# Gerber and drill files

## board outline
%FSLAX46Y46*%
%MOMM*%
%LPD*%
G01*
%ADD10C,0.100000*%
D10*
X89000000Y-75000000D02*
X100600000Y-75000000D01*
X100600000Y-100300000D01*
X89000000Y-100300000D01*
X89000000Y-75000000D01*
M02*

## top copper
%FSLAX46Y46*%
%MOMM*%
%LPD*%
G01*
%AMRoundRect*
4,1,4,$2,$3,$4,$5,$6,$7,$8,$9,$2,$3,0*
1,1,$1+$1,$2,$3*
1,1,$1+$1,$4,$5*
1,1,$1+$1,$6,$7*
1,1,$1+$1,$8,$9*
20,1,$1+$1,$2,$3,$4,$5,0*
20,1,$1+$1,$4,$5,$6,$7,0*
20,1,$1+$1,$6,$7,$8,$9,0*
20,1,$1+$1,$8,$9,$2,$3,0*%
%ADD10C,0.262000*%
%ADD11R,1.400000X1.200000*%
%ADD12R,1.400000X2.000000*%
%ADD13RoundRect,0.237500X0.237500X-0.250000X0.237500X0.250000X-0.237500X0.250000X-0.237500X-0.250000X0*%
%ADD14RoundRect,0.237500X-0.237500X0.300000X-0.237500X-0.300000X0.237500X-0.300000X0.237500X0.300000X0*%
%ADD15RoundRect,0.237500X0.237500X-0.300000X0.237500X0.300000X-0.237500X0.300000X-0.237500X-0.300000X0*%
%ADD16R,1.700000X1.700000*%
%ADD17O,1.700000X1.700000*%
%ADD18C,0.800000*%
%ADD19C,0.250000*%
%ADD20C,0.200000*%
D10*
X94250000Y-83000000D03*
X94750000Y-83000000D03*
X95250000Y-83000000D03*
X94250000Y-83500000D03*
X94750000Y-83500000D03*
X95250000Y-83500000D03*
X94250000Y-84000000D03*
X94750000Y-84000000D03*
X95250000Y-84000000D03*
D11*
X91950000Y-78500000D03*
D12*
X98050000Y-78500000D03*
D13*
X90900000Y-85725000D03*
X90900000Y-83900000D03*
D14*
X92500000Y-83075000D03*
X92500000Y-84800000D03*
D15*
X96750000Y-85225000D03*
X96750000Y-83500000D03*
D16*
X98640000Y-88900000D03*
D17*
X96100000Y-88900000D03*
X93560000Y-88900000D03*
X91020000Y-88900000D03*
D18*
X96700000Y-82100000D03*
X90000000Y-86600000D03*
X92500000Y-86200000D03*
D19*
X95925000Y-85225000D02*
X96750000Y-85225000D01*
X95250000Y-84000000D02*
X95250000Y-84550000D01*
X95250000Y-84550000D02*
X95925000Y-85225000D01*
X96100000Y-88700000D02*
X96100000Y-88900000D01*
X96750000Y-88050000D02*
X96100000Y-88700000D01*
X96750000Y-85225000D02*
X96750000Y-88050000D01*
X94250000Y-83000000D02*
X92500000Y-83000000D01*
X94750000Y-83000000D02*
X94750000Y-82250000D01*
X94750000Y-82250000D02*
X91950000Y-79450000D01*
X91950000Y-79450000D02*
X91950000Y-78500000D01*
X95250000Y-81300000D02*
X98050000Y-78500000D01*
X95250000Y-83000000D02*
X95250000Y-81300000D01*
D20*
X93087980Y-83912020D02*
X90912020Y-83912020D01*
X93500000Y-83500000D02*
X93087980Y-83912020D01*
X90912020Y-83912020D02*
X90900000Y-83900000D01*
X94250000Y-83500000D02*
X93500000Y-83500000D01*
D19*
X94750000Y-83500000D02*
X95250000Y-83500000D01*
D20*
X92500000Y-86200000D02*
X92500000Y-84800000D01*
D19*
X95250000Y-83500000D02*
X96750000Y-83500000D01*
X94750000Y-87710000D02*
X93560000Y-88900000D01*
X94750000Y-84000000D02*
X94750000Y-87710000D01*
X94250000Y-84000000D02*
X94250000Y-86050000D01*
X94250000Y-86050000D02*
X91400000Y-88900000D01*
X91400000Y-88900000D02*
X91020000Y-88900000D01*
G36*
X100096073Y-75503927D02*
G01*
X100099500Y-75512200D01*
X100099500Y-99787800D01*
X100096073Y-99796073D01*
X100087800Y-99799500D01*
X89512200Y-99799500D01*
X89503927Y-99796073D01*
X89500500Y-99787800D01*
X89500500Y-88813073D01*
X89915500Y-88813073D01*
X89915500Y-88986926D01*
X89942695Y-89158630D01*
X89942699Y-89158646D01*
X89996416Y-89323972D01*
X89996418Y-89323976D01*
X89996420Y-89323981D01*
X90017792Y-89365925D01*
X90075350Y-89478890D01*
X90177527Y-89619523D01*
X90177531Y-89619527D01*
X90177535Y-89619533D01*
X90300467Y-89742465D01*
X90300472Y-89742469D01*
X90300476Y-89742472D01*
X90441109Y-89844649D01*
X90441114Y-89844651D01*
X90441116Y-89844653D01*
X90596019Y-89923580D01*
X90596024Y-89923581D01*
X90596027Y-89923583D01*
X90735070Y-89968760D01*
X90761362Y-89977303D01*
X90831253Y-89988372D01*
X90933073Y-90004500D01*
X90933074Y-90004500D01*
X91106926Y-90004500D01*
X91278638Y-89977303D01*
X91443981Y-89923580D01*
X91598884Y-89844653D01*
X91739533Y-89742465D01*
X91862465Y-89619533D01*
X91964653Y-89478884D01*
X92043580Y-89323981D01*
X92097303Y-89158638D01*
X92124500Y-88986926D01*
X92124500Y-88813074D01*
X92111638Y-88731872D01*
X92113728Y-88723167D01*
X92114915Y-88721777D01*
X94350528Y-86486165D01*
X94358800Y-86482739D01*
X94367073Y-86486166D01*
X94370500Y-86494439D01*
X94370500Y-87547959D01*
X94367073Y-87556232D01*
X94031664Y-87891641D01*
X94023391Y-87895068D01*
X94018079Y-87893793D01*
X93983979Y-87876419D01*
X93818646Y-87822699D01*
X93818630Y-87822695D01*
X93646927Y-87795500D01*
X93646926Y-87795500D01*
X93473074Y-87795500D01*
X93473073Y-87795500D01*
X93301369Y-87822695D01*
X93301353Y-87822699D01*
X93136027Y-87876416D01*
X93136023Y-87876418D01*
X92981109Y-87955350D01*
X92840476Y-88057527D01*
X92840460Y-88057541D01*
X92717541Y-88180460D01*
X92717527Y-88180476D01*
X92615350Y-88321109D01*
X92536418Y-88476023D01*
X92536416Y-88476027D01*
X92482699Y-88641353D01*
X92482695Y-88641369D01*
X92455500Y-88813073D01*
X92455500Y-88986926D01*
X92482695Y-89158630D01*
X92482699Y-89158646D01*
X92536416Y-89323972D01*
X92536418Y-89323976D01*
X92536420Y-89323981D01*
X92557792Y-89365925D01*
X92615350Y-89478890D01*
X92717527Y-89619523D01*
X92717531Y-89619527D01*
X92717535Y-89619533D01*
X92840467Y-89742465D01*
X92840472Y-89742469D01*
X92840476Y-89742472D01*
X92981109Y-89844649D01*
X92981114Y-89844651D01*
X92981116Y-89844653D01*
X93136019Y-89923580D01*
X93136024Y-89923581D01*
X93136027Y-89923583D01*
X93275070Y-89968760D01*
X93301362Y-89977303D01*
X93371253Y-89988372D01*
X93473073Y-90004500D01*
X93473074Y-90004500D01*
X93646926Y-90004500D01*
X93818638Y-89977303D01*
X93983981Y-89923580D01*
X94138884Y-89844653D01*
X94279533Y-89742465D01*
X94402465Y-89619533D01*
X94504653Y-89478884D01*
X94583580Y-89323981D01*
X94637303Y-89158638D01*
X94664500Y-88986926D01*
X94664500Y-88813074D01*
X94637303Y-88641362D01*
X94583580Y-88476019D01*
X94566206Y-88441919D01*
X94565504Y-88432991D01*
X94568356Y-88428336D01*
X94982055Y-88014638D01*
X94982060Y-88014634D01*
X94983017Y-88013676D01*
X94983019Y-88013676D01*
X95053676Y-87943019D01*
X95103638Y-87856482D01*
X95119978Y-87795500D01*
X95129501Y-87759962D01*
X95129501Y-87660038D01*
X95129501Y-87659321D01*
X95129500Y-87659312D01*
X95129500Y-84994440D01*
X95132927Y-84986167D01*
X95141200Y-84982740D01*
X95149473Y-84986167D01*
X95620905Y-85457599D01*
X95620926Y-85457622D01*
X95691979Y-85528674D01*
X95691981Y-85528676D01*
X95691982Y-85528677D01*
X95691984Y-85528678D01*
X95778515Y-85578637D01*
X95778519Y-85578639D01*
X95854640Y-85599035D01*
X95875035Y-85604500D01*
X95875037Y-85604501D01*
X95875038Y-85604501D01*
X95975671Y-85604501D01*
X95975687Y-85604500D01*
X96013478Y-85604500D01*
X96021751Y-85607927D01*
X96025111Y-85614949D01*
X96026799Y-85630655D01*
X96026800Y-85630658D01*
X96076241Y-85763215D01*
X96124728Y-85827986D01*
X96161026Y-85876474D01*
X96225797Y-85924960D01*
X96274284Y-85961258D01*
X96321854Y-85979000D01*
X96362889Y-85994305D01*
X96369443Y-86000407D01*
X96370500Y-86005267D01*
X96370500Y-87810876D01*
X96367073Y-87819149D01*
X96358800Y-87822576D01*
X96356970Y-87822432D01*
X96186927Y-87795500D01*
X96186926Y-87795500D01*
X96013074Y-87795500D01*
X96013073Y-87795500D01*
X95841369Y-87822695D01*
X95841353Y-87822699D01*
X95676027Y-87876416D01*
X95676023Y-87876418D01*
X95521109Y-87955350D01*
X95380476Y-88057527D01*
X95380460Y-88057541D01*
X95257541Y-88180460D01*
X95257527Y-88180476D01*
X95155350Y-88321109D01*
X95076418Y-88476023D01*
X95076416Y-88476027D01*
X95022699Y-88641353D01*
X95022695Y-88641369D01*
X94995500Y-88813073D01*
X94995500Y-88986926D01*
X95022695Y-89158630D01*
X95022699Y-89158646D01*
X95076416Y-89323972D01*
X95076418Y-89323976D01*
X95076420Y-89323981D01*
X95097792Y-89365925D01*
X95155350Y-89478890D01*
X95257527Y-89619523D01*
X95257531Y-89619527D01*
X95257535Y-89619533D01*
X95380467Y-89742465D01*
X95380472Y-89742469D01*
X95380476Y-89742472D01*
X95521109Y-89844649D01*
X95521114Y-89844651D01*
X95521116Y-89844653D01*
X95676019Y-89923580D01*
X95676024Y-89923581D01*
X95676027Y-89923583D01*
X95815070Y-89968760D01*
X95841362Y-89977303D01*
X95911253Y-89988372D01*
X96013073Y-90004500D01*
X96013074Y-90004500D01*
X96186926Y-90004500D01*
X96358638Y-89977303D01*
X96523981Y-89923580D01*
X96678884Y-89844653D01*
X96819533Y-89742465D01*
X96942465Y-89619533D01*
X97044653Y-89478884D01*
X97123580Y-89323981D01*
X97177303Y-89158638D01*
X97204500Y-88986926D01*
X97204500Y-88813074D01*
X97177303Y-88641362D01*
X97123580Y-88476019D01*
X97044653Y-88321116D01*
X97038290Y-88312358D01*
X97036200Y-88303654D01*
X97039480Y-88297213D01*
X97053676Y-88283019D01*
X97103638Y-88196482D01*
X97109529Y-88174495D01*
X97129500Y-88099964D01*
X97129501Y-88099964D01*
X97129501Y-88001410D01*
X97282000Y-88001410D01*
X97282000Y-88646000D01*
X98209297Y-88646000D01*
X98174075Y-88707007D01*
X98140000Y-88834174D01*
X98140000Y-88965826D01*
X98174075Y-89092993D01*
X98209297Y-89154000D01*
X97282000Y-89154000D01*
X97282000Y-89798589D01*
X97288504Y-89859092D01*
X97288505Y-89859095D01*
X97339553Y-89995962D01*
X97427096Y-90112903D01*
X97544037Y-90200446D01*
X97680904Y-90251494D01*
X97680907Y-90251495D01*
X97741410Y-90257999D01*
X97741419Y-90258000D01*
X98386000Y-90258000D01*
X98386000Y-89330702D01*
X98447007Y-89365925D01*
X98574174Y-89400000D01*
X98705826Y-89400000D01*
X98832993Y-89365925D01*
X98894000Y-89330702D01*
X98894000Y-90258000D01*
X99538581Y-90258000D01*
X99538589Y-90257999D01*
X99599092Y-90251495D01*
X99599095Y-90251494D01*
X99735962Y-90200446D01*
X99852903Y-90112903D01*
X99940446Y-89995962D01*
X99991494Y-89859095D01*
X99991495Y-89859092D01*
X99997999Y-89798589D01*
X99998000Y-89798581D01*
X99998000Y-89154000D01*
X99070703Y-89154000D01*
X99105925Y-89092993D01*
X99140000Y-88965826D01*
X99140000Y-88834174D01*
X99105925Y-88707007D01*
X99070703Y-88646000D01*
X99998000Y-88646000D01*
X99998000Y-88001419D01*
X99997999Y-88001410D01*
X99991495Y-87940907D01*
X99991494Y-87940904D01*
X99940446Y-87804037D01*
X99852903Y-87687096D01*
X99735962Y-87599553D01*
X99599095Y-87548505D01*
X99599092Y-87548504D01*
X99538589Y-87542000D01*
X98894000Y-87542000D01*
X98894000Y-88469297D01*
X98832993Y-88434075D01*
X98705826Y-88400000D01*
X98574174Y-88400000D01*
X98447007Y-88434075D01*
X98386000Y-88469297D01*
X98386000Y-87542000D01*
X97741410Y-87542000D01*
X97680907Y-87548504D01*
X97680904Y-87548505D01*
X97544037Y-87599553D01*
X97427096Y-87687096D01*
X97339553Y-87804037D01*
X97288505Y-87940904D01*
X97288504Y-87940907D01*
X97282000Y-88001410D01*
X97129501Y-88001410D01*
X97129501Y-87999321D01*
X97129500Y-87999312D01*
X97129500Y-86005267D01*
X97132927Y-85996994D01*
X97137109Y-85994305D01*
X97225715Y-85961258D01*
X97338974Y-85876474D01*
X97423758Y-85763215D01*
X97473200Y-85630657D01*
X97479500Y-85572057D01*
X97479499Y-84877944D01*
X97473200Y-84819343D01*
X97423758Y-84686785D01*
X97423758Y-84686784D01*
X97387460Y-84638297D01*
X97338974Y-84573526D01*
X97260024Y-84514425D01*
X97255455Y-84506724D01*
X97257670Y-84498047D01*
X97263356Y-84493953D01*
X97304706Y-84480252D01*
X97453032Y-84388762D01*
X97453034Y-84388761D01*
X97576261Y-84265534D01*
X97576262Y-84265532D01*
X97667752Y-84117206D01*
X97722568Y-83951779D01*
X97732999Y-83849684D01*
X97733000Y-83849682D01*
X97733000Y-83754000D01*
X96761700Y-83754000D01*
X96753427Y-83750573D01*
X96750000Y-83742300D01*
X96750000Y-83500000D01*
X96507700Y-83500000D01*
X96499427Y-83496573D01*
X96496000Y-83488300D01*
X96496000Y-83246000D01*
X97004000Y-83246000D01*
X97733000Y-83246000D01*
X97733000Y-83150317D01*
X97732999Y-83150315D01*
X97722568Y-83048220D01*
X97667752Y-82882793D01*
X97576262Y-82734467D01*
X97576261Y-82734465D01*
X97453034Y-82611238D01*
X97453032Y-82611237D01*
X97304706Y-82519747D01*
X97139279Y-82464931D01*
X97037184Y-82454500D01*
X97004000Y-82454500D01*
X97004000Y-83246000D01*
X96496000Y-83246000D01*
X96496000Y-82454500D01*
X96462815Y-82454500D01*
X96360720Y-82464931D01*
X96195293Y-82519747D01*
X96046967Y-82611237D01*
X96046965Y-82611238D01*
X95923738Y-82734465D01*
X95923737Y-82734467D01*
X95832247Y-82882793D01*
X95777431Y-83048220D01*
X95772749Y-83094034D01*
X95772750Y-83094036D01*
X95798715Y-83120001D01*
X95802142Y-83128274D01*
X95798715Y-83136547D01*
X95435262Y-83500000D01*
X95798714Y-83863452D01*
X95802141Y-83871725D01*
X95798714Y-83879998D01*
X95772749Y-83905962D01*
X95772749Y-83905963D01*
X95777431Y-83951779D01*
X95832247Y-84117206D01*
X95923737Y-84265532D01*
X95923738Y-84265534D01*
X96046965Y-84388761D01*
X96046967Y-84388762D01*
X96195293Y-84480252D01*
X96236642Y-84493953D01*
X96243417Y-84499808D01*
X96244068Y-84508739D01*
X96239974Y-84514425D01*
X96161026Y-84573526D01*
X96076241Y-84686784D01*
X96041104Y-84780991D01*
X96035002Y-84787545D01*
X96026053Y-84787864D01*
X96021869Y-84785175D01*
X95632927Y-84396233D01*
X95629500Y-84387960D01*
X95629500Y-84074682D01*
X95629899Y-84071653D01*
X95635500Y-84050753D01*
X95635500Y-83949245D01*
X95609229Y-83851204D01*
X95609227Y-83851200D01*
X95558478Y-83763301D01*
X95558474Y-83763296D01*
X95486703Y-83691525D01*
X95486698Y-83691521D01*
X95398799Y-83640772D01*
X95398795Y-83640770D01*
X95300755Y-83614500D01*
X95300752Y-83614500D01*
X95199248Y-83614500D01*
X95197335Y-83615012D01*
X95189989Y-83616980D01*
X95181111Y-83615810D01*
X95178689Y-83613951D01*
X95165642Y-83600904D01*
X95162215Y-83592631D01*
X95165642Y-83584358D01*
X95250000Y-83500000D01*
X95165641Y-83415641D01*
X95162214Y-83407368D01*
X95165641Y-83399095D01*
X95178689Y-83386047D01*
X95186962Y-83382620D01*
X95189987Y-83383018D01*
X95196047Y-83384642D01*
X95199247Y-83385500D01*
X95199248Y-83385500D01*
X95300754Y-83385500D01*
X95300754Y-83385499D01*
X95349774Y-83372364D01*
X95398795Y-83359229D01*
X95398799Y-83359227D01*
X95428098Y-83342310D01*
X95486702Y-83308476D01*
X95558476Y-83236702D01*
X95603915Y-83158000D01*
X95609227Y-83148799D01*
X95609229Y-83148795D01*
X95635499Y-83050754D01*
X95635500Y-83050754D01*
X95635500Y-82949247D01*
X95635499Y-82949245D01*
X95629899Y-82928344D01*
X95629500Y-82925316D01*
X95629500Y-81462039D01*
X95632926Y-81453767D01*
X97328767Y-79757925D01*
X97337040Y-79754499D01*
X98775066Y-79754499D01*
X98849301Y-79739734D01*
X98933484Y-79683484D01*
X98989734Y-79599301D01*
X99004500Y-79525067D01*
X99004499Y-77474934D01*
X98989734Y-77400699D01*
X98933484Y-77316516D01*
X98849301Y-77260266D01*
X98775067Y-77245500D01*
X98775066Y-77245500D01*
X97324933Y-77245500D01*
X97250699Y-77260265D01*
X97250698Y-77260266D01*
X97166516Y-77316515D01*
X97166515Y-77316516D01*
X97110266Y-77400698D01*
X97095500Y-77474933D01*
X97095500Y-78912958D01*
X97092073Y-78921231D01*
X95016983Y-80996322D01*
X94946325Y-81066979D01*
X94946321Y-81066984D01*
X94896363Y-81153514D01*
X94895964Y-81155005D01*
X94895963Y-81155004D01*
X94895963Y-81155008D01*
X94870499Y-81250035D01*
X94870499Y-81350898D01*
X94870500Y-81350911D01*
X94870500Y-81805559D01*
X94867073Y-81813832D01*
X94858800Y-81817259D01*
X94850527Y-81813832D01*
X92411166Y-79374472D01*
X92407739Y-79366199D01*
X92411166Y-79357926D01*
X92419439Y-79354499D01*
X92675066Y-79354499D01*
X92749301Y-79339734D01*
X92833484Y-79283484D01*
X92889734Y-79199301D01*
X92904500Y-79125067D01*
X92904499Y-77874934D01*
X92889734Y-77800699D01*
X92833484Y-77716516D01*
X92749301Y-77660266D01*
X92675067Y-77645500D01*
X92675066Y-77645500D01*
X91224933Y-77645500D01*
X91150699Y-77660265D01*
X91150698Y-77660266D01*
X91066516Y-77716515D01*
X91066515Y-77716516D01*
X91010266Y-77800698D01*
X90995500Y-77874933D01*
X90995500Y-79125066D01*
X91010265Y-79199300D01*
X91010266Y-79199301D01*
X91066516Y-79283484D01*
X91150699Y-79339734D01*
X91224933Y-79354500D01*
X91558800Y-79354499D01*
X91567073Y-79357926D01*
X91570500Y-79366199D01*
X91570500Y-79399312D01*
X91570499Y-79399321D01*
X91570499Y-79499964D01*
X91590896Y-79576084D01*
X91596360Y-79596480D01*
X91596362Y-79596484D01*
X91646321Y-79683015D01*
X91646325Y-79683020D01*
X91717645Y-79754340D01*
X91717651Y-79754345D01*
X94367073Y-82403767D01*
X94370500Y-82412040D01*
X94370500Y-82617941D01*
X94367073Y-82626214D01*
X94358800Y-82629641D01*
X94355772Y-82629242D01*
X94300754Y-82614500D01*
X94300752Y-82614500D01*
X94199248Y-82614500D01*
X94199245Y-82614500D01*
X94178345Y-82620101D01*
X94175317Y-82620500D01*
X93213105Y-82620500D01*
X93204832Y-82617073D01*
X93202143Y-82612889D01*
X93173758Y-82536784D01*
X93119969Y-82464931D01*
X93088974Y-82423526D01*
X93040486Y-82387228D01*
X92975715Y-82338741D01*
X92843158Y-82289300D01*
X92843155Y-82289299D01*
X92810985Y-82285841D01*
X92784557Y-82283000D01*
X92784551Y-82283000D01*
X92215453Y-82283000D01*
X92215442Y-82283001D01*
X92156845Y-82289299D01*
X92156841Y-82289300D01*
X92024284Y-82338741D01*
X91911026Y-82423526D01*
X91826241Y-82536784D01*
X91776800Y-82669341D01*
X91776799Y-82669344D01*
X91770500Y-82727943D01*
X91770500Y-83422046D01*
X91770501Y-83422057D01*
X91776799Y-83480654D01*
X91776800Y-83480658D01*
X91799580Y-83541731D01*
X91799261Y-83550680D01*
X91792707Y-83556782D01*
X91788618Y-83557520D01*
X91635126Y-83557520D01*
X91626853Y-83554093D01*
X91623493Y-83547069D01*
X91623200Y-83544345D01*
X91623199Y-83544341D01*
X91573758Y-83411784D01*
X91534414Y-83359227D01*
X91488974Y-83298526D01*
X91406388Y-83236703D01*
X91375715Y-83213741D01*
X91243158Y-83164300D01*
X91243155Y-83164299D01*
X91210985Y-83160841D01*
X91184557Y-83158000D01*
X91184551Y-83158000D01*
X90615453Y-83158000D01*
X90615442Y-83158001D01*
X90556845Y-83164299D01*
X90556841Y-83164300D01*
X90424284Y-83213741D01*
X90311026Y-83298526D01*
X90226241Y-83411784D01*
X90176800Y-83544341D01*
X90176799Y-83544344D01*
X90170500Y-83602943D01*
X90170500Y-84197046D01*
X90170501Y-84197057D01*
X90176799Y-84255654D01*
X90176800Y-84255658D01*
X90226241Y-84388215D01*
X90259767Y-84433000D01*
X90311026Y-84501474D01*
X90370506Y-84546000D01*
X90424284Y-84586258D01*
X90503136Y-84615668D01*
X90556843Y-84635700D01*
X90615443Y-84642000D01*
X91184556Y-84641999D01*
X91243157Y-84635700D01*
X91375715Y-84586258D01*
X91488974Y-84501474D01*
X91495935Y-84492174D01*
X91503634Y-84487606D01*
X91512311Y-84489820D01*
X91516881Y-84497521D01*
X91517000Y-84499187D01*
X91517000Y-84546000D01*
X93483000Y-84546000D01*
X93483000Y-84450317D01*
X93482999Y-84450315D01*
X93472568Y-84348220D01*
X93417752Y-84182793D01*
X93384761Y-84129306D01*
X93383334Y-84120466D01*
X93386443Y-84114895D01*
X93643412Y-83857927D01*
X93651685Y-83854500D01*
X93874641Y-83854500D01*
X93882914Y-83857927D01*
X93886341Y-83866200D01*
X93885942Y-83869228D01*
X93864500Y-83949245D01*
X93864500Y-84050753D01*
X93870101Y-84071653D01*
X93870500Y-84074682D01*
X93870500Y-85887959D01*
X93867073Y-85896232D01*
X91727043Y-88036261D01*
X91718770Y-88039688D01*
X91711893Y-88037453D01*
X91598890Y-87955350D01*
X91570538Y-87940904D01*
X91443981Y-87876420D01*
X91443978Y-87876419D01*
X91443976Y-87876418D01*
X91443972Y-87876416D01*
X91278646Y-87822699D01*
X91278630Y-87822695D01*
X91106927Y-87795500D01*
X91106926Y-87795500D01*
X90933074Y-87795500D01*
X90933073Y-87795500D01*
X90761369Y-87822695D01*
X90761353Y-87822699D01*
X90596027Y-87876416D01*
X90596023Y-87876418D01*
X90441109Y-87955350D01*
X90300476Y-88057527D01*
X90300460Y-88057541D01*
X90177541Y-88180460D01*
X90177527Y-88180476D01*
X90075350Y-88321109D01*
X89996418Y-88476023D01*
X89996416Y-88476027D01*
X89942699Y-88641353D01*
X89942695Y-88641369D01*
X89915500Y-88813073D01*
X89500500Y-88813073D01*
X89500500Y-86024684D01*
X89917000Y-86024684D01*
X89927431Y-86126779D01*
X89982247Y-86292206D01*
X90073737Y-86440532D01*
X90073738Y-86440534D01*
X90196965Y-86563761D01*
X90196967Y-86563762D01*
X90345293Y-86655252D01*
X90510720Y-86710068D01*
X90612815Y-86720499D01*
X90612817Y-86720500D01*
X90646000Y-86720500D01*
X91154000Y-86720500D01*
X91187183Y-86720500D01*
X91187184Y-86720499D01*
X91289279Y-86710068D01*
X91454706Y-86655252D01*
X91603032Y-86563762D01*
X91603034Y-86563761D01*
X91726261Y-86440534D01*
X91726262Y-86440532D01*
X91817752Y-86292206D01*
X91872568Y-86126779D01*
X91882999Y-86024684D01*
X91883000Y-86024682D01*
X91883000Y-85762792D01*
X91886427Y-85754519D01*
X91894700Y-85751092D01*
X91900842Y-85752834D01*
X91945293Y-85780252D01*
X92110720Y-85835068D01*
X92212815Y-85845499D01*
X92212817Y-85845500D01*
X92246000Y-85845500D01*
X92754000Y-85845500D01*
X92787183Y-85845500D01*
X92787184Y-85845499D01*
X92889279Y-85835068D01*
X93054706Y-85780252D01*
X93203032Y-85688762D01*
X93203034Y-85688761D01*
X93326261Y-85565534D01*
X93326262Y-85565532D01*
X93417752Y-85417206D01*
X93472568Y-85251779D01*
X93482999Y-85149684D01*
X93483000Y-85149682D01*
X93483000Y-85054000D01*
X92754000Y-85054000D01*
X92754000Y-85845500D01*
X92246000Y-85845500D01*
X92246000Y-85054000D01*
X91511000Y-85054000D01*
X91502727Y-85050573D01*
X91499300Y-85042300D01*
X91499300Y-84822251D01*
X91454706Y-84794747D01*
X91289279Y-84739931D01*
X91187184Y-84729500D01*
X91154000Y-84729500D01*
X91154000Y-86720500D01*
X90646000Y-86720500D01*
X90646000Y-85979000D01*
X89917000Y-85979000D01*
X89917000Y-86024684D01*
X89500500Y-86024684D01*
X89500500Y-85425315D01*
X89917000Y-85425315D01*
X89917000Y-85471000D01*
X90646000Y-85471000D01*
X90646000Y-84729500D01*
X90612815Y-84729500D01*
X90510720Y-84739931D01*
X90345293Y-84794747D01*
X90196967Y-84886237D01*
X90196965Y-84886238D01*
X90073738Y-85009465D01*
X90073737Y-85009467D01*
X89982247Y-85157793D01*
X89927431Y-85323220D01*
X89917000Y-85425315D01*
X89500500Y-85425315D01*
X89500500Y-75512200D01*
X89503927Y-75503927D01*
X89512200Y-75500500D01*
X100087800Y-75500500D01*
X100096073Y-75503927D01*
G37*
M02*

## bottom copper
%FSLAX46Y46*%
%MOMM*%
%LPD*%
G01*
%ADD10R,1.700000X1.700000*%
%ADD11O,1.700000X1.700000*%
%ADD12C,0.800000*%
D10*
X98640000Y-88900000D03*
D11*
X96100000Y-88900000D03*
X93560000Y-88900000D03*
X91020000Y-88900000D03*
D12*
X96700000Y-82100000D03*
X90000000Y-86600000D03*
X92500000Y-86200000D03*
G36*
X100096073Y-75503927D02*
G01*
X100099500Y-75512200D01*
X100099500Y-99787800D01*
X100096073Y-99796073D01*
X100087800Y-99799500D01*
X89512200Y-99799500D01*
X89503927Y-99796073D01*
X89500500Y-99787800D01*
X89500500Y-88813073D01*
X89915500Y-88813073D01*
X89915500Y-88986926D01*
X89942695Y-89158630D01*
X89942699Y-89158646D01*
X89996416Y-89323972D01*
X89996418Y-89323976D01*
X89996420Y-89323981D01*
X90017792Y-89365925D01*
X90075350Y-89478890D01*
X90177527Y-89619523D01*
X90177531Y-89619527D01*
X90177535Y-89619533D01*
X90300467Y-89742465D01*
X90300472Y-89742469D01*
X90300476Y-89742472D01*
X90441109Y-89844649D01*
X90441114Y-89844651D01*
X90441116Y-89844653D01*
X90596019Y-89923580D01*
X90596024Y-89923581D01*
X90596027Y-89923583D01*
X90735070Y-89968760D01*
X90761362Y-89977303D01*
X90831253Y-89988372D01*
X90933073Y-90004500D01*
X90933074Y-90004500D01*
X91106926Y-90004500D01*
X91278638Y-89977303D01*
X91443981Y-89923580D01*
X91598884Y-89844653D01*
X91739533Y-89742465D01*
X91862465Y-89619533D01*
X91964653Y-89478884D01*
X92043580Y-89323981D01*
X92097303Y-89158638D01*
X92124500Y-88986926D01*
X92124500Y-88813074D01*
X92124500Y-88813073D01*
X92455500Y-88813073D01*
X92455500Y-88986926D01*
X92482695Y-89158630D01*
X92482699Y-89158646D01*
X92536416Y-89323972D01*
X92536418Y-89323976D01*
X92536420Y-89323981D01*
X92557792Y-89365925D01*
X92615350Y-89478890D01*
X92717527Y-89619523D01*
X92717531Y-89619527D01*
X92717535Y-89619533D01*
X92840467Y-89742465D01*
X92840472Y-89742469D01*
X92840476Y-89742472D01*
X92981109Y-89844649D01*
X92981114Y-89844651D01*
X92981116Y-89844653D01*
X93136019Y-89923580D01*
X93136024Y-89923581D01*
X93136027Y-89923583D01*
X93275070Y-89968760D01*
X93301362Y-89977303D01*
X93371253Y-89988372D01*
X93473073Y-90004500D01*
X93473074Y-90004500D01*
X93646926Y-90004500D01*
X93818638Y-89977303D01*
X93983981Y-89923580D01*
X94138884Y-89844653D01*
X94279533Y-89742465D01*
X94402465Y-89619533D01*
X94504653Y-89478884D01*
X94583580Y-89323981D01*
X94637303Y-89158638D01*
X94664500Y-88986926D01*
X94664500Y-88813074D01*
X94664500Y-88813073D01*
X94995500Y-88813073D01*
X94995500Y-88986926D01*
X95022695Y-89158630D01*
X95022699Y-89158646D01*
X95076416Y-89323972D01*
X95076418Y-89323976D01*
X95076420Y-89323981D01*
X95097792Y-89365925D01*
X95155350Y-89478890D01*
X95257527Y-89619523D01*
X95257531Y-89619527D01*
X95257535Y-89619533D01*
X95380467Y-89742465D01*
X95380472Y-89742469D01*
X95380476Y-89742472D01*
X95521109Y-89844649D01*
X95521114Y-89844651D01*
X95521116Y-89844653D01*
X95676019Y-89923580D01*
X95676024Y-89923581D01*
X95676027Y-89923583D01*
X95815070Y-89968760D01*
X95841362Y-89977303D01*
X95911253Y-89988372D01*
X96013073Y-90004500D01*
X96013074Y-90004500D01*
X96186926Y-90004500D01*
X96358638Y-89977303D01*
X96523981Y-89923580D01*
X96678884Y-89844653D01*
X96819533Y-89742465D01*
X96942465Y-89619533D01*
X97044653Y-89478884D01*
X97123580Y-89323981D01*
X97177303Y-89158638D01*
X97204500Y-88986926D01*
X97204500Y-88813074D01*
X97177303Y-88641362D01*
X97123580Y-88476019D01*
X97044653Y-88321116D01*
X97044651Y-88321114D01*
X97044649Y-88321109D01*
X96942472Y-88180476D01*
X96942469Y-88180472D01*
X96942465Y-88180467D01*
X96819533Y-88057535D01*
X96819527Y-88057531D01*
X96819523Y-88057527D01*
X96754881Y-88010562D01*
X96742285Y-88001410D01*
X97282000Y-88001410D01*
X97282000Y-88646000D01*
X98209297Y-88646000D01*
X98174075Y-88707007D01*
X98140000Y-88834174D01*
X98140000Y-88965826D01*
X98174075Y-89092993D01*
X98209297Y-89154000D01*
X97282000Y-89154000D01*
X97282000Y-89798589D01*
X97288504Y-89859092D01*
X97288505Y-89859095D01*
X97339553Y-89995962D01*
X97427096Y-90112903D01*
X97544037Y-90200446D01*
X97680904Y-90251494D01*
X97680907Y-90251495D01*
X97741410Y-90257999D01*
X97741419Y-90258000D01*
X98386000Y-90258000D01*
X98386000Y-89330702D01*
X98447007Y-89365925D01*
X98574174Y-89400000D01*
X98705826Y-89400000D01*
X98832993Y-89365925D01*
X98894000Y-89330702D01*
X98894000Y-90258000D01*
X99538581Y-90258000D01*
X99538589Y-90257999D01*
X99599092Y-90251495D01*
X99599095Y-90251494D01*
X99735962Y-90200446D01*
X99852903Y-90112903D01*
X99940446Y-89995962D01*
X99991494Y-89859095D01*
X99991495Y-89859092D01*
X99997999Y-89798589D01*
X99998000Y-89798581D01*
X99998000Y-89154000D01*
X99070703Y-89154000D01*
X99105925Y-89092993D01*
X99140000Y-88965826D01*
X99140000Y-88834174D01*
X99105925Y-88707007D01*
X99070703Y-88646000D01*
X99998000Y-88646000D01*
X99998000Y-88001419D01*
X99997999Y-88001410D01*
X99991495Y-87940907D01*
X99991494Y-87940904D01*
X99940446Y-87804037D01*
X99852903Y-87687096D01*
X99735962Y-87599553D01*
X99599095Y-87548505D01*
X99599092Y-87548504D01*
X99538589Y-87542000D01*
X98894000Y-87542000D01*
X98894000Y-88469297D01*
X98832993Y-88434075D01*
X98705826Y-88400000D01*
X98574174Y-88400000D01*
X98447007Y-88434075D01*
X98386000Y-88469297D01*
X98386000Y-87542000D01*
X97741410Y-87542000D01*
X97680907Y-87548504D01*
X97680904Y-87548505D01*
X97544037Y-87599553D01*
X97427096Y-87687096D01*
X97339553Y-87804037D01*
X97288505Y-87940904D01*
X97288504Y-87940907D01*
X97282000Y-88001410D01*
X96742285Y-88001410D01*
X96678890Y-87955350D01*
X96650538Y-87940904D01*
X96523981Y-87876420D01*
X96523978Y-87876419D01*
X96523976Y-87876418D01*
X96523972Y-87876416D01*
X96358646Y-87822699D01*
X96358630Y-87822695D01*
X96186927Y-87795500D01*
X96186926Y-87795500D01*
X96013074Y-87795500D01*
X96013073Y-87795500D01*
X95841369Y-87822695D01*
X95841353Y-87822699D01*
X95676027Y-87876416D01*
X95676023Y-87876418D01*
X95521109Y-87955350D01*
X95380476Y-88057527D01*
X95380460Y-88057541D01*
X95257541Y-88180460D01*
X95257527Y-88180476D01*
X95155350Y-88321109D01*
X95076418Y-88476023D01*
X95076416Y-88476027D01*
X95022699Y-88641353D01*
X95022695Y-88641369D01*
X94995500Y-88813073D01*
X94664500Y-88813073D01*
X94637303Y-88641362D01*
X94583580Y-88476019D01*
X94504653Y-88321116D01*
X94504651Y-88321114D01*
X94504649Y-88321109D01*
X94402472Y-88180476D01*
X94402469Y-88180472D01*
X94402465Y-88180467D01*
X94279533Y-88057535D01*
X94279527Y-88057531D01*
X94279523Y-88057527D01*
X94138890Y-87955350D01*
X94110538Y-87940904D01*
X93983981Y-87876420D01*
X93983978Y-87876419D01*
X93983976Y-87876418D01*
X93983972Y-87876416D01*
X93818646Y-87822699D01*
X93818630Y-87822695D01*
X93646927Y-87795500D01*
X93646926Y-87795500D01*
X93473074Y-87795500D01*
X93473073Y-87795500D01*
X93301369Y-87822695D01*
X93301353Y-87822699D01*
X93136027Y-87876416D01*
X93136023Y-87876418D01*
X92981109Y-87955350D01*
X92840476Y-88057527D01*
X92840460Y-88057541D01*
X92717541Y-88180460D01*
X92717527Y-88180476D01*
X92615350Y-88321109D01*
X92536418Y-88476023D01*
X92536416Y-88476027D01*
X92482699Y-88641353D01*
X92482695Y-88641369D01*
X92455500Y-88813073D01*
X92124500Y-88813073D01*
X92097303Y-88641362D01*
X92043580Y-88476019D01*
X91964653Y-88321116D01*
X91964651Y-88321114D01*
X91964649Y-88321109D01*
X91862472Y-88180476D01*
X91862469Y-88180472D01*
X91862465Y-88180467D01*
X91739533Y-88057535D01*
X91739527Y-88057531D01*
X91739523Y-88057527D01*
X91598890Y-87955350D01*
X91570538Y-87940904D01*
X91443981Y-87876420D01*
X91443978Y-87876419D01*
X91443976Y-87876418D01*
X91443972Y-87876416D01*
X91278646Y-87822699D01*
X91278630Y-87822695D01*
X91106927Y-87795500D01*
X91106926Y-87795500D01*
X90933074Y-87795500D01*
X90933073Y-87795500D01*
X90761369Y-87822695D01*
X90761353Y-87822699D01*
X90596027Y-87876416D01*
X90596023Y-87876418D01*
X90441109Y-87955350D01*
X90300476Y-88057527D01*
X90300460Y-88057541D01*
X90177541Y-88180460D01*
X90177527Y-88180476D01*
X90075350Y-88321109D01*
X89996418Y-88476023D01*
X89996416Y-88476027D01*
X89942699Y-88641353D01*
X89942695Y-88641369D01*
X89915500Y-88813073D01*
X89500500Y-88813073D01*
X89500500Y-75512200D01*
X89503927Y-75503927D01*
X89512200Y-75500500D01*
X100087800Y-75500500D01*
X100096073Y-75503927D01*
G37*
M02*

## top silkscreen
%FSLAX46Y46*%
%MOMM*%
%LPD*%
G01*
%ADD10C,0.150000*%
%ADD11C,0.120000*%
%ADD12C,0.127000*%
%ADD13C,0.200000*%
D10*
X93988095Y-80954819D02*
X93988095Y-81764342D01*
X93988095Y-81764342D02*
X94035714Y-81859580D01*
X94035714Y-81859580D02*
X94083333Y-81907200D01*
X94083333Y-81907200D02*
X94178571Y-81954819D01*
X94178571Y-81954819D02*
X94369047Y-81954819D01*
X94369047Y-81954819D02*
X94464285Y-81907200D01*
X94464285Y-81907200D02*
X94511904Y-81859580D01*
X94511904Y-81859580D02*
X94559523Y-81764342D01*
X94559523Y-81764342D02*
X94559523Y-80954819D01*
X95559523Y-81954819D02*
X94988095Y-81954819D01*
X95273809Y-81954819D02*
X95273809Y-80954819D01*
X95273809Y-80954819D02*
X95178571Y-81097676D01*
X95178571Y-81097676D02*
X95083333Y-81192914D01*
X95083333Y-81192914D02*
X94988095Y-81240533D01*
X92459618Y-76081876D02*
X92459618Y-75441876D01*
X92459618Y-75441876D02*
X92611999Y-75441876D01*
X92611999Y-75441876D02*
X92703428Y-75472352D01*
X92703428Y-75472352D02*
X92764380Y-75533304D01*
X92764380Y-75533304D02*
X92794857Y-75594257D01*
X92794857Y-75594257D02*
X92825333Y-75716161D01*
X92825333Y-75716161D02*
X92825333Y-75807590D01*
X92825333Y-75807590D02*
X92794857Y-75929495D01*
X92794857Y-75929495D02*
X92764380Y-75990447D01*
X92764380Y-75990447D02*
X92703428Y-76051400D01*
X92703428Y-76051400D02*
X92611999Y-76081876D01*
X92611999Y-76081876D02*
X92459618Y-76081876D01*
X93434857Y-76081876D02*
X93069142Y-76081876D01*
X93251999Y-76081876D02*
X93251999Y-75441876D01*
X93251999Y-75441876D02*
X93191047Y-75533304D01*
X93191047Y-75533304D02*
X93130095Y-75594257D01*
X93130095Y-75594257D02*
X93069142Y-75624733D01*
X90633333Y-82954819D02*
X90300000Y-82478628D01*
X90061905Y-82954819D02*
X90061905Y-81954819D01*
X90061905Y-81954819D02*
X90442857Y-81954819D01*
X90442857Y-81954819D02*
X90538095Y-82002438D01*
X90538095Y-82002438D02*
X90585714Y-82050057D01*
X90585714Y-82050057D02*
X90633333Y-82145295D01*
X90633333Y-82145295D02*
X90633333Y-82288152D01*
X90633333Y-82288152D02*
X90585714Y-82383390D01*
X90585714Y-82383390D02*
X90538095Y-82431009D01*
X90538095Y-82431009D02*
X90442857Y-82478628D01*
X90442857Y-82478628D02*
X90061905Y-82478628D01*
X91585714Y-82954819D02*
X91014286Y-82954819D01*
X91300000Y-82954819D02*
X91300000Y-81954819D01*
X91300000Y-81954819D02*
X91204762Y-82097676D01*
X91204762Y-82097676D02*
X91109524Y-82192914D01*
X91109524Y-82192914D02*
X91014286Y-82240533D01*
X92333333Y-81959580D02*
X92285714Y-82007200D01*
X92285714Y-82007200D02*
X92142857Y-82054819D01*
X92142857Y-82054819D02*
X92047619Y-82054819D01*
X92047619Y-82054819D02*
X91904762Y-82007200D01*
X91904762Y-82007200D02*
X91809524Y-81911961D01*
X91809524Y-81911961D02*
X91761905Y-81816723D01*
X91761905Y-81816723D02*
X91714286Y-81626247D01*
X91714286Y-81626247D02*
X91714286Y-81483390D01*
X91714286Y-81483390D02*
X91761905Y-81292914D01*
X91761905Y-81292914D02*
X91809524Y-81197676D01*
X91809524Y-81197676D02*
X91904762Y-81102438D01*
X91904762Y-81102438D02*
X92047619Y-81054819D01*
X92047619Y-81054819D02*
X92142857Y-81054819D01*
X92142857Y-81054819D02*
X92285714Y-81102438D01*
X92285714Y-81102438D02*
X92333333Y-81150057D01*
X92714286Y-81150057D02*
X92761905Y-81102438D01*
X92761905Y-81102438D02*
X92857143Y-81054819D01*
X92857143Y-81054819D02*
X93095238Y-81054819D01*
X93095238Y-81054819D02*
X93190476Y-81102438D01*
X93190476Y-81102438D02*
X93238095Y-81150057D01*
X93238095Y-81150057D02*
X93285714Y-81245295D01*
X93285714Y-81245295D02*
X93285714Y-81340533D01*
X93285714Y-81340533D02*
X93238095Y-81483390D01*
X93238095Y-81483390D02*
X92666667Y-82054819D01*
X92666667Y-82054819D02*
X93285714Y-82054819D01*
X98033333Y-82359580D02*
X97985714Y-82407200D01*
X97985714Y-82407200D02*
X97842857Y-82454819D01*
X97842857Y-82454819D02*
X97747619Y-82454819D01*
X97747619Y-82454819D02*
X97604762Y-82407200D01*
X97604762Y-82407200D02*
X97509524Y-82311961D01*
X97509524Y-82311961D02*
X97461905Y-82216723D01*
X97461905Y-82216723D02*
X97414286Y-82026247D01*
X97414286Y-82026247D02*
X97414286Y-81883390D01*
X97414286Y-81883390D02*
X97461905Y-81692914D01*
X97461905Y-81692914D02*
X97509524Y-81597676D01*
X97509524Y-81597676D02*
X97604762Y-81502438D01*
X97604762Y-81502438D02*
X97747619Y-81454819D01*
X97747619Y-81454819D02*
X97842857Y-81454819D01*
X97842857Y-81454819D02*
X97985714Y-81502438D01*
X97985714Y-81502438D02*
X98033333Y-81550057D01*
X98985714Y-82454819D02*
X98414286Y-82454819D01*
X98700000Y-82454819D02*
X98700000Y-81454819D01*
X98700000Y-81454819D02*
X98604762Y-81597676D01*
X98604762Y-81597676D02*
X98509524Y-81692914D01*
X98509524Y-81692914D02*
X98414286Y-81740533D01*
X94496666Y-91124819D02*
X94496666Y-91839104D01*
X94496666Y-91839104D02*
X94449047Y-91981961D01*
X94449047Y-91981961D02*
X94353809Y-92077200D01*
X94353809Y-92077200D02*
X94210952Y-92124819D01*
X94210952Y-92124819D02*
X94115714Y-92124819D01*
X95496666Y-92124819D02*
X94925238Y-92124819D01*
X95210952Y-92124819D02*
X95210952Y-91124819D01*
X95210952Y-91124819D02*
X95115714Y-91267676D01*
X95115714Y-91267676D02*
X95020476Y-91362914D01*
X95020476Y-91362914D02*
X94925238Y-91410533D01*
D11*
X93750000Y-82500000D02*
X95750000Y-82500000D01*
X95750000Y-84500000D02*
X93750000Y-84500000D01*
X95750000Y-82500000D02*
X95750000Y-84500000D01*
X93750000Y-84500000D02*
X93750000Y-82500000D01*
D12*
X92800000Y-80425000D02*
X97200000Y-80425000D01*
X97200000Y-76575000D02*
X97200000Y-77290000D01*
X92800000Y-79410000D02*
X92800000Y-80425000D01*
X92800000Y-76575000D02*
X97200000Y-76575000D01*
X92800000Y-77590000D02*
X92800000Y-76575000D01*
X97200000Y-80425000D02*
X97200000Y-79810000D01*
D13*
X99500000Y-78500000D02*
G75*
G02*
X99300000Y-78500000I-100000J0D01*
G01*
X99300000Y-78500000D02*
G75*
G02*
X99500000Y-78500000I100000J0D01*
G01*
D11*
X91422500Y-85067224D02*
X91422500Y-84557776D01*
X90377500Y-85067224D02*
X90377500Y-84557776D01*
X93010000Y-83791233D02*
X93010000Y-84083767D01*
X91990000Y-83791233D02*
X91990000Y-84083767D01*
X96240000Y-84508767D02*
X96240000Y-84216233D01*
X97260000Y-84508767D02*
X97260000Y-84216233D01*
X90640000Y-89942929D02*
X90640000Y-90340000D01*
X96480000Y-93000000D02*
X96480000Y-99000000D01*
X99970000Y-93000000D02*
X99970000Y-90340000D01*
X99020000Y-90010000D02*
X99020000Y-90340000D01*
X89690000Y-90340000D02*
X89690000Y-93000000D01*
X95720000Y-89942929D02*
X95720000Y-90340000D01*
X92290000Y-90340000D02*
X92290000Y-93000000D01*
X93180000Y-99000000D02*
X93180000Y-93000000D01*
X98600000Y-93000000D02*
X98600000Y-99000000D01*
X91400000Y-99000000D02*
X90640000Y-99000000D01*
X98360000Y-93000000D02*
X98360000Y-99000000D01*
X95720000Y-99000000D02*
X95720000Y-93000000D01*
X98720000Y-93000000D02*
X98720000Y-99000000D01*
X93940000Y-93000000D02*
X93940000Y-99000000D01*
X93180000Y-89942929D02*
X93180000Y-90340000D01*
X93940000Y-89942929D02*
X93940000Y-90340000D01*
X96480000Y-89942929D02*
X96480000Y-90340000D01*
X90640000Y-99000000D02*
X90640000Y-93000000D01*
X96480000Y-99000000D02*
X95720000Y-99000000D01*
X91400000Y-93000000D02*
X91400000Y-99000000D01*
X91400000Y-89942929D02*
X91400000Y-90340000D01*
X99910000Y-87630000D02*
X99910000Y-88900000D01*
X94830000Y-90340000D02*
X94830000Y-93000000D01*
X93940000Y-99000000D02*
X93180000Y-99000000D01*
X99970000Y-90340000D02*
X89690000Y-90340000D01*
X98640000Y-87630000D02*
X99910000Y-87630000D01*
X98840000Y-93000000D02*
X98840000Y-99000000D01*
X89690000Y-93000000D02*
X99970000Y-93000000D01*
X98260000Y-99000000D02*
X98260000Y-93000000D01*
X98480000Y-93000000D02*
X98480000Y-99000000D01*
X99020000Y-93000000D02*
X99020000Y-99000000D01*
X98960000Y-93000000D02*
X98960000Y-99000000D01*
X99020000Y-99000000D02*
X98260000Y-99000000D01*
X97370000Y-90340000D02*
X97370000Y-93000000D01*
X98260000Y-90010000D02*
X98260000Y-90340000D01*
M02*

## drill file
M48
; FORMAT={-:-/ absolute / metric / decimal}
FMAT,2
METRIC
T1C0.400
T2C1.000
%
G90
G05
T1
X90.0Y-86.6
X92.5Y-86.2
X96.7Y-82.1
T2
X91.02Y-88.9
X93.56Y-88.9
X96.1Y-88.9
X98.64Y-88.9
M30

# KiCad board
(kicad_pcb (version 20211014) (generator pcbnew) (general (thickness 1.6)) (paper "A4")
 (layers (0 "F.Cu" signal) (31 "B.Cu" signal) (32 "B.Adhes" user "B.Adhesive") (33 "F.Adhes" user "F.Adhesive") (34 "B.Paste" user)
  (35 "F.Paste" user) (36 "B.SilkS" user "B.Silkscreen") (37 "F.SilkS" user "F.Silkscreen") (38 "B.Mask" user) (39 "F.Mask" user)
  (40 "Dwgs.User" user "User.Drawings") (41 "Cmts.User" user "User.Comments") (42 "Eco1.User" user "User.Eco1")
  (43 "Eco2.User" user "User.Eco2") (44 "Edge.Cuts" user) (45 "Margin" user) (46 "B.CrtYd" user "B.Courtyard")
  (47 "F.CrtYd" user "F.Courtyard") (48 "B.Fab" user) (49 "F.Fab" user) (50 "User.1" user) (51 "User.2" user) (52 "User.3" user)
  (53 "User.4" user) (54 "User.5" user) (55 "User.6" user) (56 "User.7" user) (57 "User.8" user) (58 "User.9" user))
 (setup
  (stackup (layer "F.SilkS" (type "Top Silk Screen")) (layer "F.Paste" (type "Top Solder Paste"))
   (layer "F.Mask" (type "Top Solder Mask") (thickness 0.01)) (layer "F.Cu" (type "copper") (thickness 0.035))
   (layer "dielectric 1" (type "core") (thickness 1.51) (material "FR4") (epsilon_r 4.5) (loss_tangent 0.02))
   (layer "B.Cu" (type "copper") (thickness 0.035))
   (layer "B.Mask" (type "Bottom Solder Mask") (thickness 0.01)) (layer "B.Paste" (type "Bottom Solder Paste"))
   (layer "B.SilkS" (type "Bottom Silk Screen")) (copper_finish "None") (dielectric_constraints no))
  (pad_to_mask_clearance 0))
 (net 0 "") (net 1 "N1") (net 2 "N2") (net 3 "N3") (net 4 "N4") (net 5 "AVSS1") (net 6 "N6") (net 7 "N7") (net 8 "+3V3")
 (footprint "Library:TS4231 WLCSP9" (layer "F.Cu") (at 94.75 83.5)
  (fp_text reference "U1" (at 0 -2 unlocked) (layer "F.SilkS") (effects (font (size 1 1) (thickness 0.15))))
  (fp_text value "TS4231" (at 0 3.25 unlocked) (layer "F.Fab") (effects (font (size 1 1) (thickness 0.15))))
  (fp_line (start -1 -1) (end 1 -1) (layer "F.SilkS") (width 0.12))
  (fp_line (start 1 1) (end -1 1) (layer "F.SilkS") (width 0.12))
  (fp_line (start 1 -1) (end 1 1) (layer "F.SilkS") (width 0.12))
  (fp_line (start -1 1) (end -1 -1) (layer "F.SilkS") (width 0.12))
  (pad "A1" smd circle (at -0.5 -0.5) (size 0.262 0.262) (layers "F.Cu" "F.Paste" "F.Mask") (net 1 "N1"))
  (pad "A2" smd circle (at 0 -0.5) (size 0.262 0.262) (layers "F.Cu" "F.Paste" "F.Mask") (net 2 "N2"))
  (pad "A3" smd circle (at 0.5 -0.5) (size 0.262 0.262) (layers "F.Cu" "F.Paste" "F.Mask") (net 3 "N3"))
  (pad "B1" smd circle (at -0.5 0) (size 0.262 0.262) (layers "F.Cu" "F.Paste" "F.Mask") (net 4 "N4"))
  (pad "B2" smd circle (at 0 0) (size 0.262 0.262) (layers "F.Cu" "F.Paste" "F.Mask") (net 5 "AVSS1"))
  (pad "B3" smd circle (at 0.5 0) (size 0.262 0.262) (layers "F.Cu" "F.Paste" "F.Mask") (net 5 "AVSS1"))
  (pad "C1" smd circle (at -0.5 0.5) (size 0.262 0.262) (layers "F.Cu" "F.Paste" "F.Mask") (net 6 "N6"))
  (pad "C2" smd circle (at 0 0.5) (size 0.262 0.262) (layers "F.Cu" "F.Paste" "F.Mask") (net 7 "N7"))
  (pad "C3" smd circle (at 0.5 0.5) (size 0.262 0.262) (layers "F.Cu" "F.Paste" "F.Mask") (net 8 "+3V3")))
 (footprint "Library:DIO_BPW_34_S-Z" (layer "F.Cu") (at 95 78.5)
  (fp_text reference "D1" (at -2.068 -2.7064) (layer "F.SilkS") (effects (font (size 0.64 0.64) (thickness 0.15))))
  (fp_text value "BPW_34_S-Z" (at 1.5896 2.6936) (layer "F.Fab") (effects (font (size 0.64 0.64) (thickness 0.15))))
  (fp_line (start -2.2 1.925) (end 2.2 1.925) (layer "F.SilkS") (width 0.127))
  (fp_line (start 2.2 -1.925) (end 2.2 -1.21) (layer "F.SilkS") (width 0.127))
  (fp_line (start -2.2 0.91) (end -2.2 1.925) (layer "F.SilkS") (width 0.127))
  (fp_line (start -2.2 -1.925) (end 2.2 -1.925) (layer "F.SilkS") (width 0.127))
  (fp_line (start -2.2 -0.91) (end -2.2 -1.925) (layer "F.SilkS") (width 0.127))
  (fp_line (start 2.2 1.925) (end 2.2 1.31) (layer "F.SilkS") (width 0.127))
  (fp_circle (center 4.4 0) (end 4.5 0) (layer "F.SilkS") (width 0.2) (fill none))
  (pad "A" smd rect (at -3.05 0 90) (size 1.2 1.4) (layers "F.Cu") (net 2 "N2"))
  (pad "C" smd rect (at 3.05 0 90) (size 2 1.4) (layers "F.Cu") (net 3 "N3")))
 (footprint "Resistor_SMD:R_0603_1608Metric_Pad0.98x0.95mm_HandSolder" (layer "F.Cu") (at 90.9 84.8125 90)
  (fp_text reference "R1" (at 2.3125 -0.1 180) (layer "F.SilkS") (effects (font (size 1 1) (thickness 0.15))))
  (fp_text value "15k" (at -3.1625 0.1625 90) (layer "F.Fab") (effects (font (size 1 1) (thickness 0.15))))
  (fp_line (start -0.254724 0.5225) (end 0.254724 0.5225) (layer "F.SilkS") (width 0.12))
  (fp_line (start -0.254724 -0.5225) (end 0.254724 -0.5225) (layer "F.SilkS") (width 0.12))
  (pad "1" smd roundrect locked (at -0.9125 0 90) (size 0.975 0.95) (layers "F.Cu" "F.Paste" "F.Mask") (roundrect_rratio 0.25)
   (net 5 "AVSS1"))
  (pad "2" smd roundrect locked (at 0.9125 0 90) (size 0.975 0.95) (layers "F.Cu" "F.Paste" "F.Mask") (roundrect_rratio 0.25) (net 4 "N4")))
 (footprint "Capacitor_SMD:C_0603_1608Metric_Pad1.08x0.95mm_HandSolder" (layer "F.Cu") (at 92.5 83.9375 -90)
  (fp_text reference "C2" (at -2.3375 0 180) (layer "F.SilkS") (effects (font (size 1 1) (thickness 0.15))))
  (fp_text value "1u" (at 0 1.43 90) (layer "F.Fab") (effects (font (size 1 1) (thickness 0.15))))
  (fp_line (start -0.146267 -0.51) (end 0.146267 -0.51) (layer "F.SilkS") (width 0.12))
  (fp_line (start -0.146267 0.51) (end 0.146267 0.51) (layer "F.SilkS") (width 0.12))
  (pad "1" smd roundrect locked (at -0.8625 0 270) (size 1.075 0.95) (layers "F.Cu" "F.Paste" "F.Mask") (roundrect_rratio 0.25) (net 1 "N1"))
  (pad "2" smd roundrect locked (at 0.8625 0 270) (size 1.075 0.95) (layers "F.Cu" "F.Paste" "F.Mask") (roundrect_rratio 0.25)
   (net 5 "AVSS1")))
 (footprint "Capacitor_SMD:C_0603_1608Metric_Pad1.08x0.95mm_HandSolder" (layer "F.Cu") (at 96.75 84.3625 90)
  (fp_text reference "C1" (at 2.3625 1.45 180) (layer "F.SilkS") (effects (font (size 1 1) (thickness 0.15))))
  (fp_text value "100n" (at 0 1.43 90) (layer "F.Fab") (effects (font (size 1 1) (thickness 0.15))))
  (fp_line (start -0.146267 -0.51) (end 0.146267 -0.51) (layer "F.SilkS") (width 0.12))
  (fp_line (start -0.146267 0.51) (end 0.146267 0.51) (layer "F.SilkS") (width 0.12))
  (pad "1" smd roundrect locked (at -0.8625 0 90) (size 1.075 0.95) (layers "F.Cu" "F.Paste" "F.Mask") (roundrect_rratio 0.25)
   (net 8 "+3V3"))
  (pad "2" smd roundrect locked (at 0.8625 0 90) (size 1.075 0.95) (layers "F.Cu" "F.Paste" "F.Mask") (roundrect_rratio 0.25)
   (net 5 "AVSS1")))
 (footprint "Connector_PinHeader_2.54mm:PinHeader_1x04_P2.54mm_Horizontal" (layer "F.Cu") (at 98.64 88.9 -90)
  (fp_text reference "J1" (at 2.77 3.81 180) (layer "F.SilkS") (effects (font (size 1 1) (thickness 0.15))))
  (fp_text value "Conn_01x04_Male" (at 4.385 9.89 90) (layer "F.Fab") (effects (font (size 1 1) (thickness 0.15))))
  (fp_line (start 1.042929 8) (end 1.44 8) (layer "F.SilkS") (width 0.12))
  (fp_line (start 4.1 2.16) (end 10.1 2.16) (layer "F.SilkS") (width 0.12))
  (fp_line (start 4.1 -1.33) (end 1.44 -1.33) (layer "F.SilkS") (width 0.12))
  (fp_line (start 1.11 -0.38) (end 1.44 -0.38) (layer "F.SilkS") (width 0.12))
  (fp_line (start 1.44 8.95) (end 4.1 8.95) (layer "F.SilkS") (width 0.12))
  (fp_line (start 1.042929 2.92) (end 1.44 2.92) (layer "F.SilkS") (width 0.12))
  (fp_line (start 1.44 6.35) (end 4.1 6.35) (layer "F.SilkS") (width 0.12))
  (fp_line (start 10.1 5.46) (end 4.1 5.46) (layer "F.SilkS") (width 0.12))
  (fp_line (start 4.1 0.04) (end 10.1 0.04) (layer "F.SilkS") (width 0.12))
  (fp_line (start 10.1 7.24) (end 10.1 8) (layer "F.SilkS") (width 0.12))
  (fp_line (start 4.1 0.28) (end 10.1 0.28) (layer "F.SilkS") (width 0.12))
  (fp_line (start 10.1 2.92) (end 4.1 2.92) (layer "F.SilkS") (width 0.12))
  (fp_line (start 4.1 -0.08) (end 10.1 -0.08) (layer "F.SilkS") (width 0.12))
  (fp_line (start 4.1 4.7) (end 10.1 4.7) (layer "F.SilkS") (width 0.12))
  (fp_line (start 1.042929 5.46) (end 1.44 5.46) (layer "F.SilkS") (width 0.12))
  (fp_line (start 1.042929 4.7) (end 1.44 4.7) (layer "F.SilkS") (width 0.12))
  (fp_line (start 1.042929 2.16) (end 1.44 2.16) (layer "F.SilkS") (width 0.12))
  (fp_line (start 10.1 8) (end 4.1 8) (layer "F.SilkS") (width 0.12))
  (fp_line (start 10.1 2.16) (end 10.1 2.92) (layer "F.SilkS") (width 0.12))
  (fp_line (start 4.1 7.24) (end 10.1 7.24) (layer "F.SilkS") (width 0.12))
  (fp_line (start 1.042929 7.24) (end 1.44 7.24) (layer "F.SilkS") (width 0.12))
  (fp_line (start -1.27 -1.27) (end 0 -1.27) (layer "F.SilkS") (width 0.12))
  (fp_line (start 1.44 3.81) (end 4.1 3.81) (layer "F.SilkS") (width 0.12))
  (fp_line (start 10.1 4.7) (end 10.1 5.46) (layer "F.SilkS") (width 0.12))
  (fp_line (start 1.44 -1.33) (end 1.44 8.95) (layer "F.SilkS") (width 0.12))
  (fp_line (start -1.27 0) (end -1.27 -1.27) (layer "F.SilkS") (width 0.12))
  (fp_line (start 4.1 -0.2) (end 10.1 -0.2) (layer "F.SilkS") (width 0.12))
  (fp_line (start 4.1 8.95) (end 4.1 -1.33) (layer "F.SilkS") (width 0.12))
  (fp_line (start 10.1 0.38) (end 4.1 0.38) (layer "F.SilkS") (width 0.12))
  (fp_line (start 4.1 0.16) (end 10.1 0.16) (layer "F.SilkS") (width 0.12))
  (fp_line (start 4.1 -0.38) (end 10.1 -0.38) (layer "F.SilkS") (width 0.12))
  (fp_line (start 4.1 -0.32) (end 10.1 -0.32) (layer "F.SilkS") (width 0.12))
  (fp_line (start 10.1 -0.38) (end 10.1 0.38) (layer "F.SilkS") (width 0.12))
  (fp_line (start 1.44 1.27) (end 4.1 1.27) (layer "F.SilkS") (width 0.12))
  (fp_line (start 1.11 0.38) (end 1.44 0.38) (layer "F.SilkS") (width 0.12))
  (pad "1" thru_hole rect locked (at 0 0 270) (size 1.7 1.7) (drill 1) (layers *.Cu *.Mask) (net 5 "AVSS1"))
  (pad "2" thru_hole oval locked (at 0 2.54 270) (size 1.7 1.7) (drill 1) (layers *.Cu *.Mask) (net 8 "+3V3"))
  (pad "3" thru_hole oval locked (at 0 5.08 270) (size 1.7 1.7) (drill 1) (layers *.Cu *.Mask) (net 7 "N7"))
  (pad "4" thru_hole oval locked (at 0 7.62 270) (size 1.7 1.7) (drill 1) (layers *.Cu *.Mask) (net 6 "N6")))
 (gr_rect (start 89 100.3) (end 100.6 75) (layer "Edge.Cuts") (width 0.1) (fill none))
 (segment (start 95.925 85.225) (end 96.75 85.225) (width 0.25) (layer "F.Cu") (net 8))
 (segment (start 95.25 84) (end 95.25 84.55) (width 0.25) (layer "F.Cu") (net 8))
 (segment (start 95.25 84.55) (end 95.925 85.225) (width 0.25) (layer "F.Cu") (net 8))
 (segment (start 96.1 88.7) (end 96.1 88.9) (width 0.25) (layer "F.Cu") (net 8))
 (segment (start 96.75 88.05) (end 96.1 88.7) (width 0.25) (layer "F.Cu") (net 8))
 (segment (start 96.75 85.225) (end 96.75 88.05) (width 0.25) (layer "F.Cu") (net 8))
 (segment (start 94.25 83) (end 92.5 83) (width 0.25) (layer "F.Cu") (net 1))
 (segment (start 94.75 83) (end 94.75 82.25) (width 0.25) (layer "F.Cu") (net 2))
 (segment (start 94.75 82.25) (end 91.95 79.45) (width 0.25) (layer "F.Cu") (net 2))
 (segment (start 91.95 79.45) (end 91.95 78.5) (width 0.25) (layer "F.Cu") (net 2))
 (segment (start 95.25 81.3) (end 98.05 78.5) (width 0.25) (layer "F.Cu") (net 3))
 (segment (start 95.25 83) (end 95.25 81.3) (width 0.25) (layer "F.Cu") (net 3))
 (segment (start 93.08798 83.91202) (end 90.91202 83.91202) (width 0.2) (layer "F.Cu") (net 4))
 (segment (start 93.5 83.5) (end 93.08798 83.91202) (width 0.2) (layer "F.Cu") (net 4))
 (segment (start 90.91202 83.91202) (end 90.9 83.9) (width 0.2) (layer "F.Cu") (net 4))
 (segment (start 94.25 83.5) (end 93.5 83.5) (width 0.2) (layer "F.Cu") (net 4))
 (segment (start 94.75 83.5) (end 95.25 83.5) (width 0.25) (layer "F.Cu") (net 5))
 (segment (start 92.5 86.2) (end 92.5 84.8) (width 0.2) (layer "F.Cu") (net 5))
 (segment (start 95.25 83.5) (end 96.75 83.5) (width 0.25) (layer "F.Cu") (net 5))
 (via (at 96.7 82.1) (size 0.8) (drill 0.4) (layers "F.Cu" "B.Cu") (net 5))
 (via (at 90 86.6) (size 0.8) (drill 0.4) (layers "F.Cu" "B.Cu") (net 5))
 (via (at 92.5 86.2) (size 0.8) (drill 0.4) (layers "F.Cu" "B.Cu") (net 5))
 (segment (start 94.75 87.71) (end 93.56 88.9) (width 0.25) (layer "F.Cu") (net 7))
 (segment (start 94.75 84) (end 94.75 87.71) (width 0.25) (layer "F.Cu") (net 7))
 (segment (start 94.25 84) (end 94.25 86.05) (width 0.25) (layer "F.Cu") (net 6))
 (segment (start 94.25 86.05) (end 91.4 88.9) (width 0.25) (layer "F.Cu") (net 6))
 (segment (start 91.4 88.9) (end 91.02 88.9) (width 0.25) (layer "F.Cu") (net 6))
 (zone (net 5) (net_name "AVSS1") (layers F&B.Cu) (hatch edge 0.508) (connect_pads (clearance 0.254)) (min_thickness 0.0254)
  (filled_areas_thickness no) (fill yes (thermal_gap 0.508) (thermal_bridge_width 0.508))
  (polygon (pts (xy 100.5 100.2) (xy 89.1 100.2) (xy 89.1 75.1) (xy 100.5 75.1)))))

